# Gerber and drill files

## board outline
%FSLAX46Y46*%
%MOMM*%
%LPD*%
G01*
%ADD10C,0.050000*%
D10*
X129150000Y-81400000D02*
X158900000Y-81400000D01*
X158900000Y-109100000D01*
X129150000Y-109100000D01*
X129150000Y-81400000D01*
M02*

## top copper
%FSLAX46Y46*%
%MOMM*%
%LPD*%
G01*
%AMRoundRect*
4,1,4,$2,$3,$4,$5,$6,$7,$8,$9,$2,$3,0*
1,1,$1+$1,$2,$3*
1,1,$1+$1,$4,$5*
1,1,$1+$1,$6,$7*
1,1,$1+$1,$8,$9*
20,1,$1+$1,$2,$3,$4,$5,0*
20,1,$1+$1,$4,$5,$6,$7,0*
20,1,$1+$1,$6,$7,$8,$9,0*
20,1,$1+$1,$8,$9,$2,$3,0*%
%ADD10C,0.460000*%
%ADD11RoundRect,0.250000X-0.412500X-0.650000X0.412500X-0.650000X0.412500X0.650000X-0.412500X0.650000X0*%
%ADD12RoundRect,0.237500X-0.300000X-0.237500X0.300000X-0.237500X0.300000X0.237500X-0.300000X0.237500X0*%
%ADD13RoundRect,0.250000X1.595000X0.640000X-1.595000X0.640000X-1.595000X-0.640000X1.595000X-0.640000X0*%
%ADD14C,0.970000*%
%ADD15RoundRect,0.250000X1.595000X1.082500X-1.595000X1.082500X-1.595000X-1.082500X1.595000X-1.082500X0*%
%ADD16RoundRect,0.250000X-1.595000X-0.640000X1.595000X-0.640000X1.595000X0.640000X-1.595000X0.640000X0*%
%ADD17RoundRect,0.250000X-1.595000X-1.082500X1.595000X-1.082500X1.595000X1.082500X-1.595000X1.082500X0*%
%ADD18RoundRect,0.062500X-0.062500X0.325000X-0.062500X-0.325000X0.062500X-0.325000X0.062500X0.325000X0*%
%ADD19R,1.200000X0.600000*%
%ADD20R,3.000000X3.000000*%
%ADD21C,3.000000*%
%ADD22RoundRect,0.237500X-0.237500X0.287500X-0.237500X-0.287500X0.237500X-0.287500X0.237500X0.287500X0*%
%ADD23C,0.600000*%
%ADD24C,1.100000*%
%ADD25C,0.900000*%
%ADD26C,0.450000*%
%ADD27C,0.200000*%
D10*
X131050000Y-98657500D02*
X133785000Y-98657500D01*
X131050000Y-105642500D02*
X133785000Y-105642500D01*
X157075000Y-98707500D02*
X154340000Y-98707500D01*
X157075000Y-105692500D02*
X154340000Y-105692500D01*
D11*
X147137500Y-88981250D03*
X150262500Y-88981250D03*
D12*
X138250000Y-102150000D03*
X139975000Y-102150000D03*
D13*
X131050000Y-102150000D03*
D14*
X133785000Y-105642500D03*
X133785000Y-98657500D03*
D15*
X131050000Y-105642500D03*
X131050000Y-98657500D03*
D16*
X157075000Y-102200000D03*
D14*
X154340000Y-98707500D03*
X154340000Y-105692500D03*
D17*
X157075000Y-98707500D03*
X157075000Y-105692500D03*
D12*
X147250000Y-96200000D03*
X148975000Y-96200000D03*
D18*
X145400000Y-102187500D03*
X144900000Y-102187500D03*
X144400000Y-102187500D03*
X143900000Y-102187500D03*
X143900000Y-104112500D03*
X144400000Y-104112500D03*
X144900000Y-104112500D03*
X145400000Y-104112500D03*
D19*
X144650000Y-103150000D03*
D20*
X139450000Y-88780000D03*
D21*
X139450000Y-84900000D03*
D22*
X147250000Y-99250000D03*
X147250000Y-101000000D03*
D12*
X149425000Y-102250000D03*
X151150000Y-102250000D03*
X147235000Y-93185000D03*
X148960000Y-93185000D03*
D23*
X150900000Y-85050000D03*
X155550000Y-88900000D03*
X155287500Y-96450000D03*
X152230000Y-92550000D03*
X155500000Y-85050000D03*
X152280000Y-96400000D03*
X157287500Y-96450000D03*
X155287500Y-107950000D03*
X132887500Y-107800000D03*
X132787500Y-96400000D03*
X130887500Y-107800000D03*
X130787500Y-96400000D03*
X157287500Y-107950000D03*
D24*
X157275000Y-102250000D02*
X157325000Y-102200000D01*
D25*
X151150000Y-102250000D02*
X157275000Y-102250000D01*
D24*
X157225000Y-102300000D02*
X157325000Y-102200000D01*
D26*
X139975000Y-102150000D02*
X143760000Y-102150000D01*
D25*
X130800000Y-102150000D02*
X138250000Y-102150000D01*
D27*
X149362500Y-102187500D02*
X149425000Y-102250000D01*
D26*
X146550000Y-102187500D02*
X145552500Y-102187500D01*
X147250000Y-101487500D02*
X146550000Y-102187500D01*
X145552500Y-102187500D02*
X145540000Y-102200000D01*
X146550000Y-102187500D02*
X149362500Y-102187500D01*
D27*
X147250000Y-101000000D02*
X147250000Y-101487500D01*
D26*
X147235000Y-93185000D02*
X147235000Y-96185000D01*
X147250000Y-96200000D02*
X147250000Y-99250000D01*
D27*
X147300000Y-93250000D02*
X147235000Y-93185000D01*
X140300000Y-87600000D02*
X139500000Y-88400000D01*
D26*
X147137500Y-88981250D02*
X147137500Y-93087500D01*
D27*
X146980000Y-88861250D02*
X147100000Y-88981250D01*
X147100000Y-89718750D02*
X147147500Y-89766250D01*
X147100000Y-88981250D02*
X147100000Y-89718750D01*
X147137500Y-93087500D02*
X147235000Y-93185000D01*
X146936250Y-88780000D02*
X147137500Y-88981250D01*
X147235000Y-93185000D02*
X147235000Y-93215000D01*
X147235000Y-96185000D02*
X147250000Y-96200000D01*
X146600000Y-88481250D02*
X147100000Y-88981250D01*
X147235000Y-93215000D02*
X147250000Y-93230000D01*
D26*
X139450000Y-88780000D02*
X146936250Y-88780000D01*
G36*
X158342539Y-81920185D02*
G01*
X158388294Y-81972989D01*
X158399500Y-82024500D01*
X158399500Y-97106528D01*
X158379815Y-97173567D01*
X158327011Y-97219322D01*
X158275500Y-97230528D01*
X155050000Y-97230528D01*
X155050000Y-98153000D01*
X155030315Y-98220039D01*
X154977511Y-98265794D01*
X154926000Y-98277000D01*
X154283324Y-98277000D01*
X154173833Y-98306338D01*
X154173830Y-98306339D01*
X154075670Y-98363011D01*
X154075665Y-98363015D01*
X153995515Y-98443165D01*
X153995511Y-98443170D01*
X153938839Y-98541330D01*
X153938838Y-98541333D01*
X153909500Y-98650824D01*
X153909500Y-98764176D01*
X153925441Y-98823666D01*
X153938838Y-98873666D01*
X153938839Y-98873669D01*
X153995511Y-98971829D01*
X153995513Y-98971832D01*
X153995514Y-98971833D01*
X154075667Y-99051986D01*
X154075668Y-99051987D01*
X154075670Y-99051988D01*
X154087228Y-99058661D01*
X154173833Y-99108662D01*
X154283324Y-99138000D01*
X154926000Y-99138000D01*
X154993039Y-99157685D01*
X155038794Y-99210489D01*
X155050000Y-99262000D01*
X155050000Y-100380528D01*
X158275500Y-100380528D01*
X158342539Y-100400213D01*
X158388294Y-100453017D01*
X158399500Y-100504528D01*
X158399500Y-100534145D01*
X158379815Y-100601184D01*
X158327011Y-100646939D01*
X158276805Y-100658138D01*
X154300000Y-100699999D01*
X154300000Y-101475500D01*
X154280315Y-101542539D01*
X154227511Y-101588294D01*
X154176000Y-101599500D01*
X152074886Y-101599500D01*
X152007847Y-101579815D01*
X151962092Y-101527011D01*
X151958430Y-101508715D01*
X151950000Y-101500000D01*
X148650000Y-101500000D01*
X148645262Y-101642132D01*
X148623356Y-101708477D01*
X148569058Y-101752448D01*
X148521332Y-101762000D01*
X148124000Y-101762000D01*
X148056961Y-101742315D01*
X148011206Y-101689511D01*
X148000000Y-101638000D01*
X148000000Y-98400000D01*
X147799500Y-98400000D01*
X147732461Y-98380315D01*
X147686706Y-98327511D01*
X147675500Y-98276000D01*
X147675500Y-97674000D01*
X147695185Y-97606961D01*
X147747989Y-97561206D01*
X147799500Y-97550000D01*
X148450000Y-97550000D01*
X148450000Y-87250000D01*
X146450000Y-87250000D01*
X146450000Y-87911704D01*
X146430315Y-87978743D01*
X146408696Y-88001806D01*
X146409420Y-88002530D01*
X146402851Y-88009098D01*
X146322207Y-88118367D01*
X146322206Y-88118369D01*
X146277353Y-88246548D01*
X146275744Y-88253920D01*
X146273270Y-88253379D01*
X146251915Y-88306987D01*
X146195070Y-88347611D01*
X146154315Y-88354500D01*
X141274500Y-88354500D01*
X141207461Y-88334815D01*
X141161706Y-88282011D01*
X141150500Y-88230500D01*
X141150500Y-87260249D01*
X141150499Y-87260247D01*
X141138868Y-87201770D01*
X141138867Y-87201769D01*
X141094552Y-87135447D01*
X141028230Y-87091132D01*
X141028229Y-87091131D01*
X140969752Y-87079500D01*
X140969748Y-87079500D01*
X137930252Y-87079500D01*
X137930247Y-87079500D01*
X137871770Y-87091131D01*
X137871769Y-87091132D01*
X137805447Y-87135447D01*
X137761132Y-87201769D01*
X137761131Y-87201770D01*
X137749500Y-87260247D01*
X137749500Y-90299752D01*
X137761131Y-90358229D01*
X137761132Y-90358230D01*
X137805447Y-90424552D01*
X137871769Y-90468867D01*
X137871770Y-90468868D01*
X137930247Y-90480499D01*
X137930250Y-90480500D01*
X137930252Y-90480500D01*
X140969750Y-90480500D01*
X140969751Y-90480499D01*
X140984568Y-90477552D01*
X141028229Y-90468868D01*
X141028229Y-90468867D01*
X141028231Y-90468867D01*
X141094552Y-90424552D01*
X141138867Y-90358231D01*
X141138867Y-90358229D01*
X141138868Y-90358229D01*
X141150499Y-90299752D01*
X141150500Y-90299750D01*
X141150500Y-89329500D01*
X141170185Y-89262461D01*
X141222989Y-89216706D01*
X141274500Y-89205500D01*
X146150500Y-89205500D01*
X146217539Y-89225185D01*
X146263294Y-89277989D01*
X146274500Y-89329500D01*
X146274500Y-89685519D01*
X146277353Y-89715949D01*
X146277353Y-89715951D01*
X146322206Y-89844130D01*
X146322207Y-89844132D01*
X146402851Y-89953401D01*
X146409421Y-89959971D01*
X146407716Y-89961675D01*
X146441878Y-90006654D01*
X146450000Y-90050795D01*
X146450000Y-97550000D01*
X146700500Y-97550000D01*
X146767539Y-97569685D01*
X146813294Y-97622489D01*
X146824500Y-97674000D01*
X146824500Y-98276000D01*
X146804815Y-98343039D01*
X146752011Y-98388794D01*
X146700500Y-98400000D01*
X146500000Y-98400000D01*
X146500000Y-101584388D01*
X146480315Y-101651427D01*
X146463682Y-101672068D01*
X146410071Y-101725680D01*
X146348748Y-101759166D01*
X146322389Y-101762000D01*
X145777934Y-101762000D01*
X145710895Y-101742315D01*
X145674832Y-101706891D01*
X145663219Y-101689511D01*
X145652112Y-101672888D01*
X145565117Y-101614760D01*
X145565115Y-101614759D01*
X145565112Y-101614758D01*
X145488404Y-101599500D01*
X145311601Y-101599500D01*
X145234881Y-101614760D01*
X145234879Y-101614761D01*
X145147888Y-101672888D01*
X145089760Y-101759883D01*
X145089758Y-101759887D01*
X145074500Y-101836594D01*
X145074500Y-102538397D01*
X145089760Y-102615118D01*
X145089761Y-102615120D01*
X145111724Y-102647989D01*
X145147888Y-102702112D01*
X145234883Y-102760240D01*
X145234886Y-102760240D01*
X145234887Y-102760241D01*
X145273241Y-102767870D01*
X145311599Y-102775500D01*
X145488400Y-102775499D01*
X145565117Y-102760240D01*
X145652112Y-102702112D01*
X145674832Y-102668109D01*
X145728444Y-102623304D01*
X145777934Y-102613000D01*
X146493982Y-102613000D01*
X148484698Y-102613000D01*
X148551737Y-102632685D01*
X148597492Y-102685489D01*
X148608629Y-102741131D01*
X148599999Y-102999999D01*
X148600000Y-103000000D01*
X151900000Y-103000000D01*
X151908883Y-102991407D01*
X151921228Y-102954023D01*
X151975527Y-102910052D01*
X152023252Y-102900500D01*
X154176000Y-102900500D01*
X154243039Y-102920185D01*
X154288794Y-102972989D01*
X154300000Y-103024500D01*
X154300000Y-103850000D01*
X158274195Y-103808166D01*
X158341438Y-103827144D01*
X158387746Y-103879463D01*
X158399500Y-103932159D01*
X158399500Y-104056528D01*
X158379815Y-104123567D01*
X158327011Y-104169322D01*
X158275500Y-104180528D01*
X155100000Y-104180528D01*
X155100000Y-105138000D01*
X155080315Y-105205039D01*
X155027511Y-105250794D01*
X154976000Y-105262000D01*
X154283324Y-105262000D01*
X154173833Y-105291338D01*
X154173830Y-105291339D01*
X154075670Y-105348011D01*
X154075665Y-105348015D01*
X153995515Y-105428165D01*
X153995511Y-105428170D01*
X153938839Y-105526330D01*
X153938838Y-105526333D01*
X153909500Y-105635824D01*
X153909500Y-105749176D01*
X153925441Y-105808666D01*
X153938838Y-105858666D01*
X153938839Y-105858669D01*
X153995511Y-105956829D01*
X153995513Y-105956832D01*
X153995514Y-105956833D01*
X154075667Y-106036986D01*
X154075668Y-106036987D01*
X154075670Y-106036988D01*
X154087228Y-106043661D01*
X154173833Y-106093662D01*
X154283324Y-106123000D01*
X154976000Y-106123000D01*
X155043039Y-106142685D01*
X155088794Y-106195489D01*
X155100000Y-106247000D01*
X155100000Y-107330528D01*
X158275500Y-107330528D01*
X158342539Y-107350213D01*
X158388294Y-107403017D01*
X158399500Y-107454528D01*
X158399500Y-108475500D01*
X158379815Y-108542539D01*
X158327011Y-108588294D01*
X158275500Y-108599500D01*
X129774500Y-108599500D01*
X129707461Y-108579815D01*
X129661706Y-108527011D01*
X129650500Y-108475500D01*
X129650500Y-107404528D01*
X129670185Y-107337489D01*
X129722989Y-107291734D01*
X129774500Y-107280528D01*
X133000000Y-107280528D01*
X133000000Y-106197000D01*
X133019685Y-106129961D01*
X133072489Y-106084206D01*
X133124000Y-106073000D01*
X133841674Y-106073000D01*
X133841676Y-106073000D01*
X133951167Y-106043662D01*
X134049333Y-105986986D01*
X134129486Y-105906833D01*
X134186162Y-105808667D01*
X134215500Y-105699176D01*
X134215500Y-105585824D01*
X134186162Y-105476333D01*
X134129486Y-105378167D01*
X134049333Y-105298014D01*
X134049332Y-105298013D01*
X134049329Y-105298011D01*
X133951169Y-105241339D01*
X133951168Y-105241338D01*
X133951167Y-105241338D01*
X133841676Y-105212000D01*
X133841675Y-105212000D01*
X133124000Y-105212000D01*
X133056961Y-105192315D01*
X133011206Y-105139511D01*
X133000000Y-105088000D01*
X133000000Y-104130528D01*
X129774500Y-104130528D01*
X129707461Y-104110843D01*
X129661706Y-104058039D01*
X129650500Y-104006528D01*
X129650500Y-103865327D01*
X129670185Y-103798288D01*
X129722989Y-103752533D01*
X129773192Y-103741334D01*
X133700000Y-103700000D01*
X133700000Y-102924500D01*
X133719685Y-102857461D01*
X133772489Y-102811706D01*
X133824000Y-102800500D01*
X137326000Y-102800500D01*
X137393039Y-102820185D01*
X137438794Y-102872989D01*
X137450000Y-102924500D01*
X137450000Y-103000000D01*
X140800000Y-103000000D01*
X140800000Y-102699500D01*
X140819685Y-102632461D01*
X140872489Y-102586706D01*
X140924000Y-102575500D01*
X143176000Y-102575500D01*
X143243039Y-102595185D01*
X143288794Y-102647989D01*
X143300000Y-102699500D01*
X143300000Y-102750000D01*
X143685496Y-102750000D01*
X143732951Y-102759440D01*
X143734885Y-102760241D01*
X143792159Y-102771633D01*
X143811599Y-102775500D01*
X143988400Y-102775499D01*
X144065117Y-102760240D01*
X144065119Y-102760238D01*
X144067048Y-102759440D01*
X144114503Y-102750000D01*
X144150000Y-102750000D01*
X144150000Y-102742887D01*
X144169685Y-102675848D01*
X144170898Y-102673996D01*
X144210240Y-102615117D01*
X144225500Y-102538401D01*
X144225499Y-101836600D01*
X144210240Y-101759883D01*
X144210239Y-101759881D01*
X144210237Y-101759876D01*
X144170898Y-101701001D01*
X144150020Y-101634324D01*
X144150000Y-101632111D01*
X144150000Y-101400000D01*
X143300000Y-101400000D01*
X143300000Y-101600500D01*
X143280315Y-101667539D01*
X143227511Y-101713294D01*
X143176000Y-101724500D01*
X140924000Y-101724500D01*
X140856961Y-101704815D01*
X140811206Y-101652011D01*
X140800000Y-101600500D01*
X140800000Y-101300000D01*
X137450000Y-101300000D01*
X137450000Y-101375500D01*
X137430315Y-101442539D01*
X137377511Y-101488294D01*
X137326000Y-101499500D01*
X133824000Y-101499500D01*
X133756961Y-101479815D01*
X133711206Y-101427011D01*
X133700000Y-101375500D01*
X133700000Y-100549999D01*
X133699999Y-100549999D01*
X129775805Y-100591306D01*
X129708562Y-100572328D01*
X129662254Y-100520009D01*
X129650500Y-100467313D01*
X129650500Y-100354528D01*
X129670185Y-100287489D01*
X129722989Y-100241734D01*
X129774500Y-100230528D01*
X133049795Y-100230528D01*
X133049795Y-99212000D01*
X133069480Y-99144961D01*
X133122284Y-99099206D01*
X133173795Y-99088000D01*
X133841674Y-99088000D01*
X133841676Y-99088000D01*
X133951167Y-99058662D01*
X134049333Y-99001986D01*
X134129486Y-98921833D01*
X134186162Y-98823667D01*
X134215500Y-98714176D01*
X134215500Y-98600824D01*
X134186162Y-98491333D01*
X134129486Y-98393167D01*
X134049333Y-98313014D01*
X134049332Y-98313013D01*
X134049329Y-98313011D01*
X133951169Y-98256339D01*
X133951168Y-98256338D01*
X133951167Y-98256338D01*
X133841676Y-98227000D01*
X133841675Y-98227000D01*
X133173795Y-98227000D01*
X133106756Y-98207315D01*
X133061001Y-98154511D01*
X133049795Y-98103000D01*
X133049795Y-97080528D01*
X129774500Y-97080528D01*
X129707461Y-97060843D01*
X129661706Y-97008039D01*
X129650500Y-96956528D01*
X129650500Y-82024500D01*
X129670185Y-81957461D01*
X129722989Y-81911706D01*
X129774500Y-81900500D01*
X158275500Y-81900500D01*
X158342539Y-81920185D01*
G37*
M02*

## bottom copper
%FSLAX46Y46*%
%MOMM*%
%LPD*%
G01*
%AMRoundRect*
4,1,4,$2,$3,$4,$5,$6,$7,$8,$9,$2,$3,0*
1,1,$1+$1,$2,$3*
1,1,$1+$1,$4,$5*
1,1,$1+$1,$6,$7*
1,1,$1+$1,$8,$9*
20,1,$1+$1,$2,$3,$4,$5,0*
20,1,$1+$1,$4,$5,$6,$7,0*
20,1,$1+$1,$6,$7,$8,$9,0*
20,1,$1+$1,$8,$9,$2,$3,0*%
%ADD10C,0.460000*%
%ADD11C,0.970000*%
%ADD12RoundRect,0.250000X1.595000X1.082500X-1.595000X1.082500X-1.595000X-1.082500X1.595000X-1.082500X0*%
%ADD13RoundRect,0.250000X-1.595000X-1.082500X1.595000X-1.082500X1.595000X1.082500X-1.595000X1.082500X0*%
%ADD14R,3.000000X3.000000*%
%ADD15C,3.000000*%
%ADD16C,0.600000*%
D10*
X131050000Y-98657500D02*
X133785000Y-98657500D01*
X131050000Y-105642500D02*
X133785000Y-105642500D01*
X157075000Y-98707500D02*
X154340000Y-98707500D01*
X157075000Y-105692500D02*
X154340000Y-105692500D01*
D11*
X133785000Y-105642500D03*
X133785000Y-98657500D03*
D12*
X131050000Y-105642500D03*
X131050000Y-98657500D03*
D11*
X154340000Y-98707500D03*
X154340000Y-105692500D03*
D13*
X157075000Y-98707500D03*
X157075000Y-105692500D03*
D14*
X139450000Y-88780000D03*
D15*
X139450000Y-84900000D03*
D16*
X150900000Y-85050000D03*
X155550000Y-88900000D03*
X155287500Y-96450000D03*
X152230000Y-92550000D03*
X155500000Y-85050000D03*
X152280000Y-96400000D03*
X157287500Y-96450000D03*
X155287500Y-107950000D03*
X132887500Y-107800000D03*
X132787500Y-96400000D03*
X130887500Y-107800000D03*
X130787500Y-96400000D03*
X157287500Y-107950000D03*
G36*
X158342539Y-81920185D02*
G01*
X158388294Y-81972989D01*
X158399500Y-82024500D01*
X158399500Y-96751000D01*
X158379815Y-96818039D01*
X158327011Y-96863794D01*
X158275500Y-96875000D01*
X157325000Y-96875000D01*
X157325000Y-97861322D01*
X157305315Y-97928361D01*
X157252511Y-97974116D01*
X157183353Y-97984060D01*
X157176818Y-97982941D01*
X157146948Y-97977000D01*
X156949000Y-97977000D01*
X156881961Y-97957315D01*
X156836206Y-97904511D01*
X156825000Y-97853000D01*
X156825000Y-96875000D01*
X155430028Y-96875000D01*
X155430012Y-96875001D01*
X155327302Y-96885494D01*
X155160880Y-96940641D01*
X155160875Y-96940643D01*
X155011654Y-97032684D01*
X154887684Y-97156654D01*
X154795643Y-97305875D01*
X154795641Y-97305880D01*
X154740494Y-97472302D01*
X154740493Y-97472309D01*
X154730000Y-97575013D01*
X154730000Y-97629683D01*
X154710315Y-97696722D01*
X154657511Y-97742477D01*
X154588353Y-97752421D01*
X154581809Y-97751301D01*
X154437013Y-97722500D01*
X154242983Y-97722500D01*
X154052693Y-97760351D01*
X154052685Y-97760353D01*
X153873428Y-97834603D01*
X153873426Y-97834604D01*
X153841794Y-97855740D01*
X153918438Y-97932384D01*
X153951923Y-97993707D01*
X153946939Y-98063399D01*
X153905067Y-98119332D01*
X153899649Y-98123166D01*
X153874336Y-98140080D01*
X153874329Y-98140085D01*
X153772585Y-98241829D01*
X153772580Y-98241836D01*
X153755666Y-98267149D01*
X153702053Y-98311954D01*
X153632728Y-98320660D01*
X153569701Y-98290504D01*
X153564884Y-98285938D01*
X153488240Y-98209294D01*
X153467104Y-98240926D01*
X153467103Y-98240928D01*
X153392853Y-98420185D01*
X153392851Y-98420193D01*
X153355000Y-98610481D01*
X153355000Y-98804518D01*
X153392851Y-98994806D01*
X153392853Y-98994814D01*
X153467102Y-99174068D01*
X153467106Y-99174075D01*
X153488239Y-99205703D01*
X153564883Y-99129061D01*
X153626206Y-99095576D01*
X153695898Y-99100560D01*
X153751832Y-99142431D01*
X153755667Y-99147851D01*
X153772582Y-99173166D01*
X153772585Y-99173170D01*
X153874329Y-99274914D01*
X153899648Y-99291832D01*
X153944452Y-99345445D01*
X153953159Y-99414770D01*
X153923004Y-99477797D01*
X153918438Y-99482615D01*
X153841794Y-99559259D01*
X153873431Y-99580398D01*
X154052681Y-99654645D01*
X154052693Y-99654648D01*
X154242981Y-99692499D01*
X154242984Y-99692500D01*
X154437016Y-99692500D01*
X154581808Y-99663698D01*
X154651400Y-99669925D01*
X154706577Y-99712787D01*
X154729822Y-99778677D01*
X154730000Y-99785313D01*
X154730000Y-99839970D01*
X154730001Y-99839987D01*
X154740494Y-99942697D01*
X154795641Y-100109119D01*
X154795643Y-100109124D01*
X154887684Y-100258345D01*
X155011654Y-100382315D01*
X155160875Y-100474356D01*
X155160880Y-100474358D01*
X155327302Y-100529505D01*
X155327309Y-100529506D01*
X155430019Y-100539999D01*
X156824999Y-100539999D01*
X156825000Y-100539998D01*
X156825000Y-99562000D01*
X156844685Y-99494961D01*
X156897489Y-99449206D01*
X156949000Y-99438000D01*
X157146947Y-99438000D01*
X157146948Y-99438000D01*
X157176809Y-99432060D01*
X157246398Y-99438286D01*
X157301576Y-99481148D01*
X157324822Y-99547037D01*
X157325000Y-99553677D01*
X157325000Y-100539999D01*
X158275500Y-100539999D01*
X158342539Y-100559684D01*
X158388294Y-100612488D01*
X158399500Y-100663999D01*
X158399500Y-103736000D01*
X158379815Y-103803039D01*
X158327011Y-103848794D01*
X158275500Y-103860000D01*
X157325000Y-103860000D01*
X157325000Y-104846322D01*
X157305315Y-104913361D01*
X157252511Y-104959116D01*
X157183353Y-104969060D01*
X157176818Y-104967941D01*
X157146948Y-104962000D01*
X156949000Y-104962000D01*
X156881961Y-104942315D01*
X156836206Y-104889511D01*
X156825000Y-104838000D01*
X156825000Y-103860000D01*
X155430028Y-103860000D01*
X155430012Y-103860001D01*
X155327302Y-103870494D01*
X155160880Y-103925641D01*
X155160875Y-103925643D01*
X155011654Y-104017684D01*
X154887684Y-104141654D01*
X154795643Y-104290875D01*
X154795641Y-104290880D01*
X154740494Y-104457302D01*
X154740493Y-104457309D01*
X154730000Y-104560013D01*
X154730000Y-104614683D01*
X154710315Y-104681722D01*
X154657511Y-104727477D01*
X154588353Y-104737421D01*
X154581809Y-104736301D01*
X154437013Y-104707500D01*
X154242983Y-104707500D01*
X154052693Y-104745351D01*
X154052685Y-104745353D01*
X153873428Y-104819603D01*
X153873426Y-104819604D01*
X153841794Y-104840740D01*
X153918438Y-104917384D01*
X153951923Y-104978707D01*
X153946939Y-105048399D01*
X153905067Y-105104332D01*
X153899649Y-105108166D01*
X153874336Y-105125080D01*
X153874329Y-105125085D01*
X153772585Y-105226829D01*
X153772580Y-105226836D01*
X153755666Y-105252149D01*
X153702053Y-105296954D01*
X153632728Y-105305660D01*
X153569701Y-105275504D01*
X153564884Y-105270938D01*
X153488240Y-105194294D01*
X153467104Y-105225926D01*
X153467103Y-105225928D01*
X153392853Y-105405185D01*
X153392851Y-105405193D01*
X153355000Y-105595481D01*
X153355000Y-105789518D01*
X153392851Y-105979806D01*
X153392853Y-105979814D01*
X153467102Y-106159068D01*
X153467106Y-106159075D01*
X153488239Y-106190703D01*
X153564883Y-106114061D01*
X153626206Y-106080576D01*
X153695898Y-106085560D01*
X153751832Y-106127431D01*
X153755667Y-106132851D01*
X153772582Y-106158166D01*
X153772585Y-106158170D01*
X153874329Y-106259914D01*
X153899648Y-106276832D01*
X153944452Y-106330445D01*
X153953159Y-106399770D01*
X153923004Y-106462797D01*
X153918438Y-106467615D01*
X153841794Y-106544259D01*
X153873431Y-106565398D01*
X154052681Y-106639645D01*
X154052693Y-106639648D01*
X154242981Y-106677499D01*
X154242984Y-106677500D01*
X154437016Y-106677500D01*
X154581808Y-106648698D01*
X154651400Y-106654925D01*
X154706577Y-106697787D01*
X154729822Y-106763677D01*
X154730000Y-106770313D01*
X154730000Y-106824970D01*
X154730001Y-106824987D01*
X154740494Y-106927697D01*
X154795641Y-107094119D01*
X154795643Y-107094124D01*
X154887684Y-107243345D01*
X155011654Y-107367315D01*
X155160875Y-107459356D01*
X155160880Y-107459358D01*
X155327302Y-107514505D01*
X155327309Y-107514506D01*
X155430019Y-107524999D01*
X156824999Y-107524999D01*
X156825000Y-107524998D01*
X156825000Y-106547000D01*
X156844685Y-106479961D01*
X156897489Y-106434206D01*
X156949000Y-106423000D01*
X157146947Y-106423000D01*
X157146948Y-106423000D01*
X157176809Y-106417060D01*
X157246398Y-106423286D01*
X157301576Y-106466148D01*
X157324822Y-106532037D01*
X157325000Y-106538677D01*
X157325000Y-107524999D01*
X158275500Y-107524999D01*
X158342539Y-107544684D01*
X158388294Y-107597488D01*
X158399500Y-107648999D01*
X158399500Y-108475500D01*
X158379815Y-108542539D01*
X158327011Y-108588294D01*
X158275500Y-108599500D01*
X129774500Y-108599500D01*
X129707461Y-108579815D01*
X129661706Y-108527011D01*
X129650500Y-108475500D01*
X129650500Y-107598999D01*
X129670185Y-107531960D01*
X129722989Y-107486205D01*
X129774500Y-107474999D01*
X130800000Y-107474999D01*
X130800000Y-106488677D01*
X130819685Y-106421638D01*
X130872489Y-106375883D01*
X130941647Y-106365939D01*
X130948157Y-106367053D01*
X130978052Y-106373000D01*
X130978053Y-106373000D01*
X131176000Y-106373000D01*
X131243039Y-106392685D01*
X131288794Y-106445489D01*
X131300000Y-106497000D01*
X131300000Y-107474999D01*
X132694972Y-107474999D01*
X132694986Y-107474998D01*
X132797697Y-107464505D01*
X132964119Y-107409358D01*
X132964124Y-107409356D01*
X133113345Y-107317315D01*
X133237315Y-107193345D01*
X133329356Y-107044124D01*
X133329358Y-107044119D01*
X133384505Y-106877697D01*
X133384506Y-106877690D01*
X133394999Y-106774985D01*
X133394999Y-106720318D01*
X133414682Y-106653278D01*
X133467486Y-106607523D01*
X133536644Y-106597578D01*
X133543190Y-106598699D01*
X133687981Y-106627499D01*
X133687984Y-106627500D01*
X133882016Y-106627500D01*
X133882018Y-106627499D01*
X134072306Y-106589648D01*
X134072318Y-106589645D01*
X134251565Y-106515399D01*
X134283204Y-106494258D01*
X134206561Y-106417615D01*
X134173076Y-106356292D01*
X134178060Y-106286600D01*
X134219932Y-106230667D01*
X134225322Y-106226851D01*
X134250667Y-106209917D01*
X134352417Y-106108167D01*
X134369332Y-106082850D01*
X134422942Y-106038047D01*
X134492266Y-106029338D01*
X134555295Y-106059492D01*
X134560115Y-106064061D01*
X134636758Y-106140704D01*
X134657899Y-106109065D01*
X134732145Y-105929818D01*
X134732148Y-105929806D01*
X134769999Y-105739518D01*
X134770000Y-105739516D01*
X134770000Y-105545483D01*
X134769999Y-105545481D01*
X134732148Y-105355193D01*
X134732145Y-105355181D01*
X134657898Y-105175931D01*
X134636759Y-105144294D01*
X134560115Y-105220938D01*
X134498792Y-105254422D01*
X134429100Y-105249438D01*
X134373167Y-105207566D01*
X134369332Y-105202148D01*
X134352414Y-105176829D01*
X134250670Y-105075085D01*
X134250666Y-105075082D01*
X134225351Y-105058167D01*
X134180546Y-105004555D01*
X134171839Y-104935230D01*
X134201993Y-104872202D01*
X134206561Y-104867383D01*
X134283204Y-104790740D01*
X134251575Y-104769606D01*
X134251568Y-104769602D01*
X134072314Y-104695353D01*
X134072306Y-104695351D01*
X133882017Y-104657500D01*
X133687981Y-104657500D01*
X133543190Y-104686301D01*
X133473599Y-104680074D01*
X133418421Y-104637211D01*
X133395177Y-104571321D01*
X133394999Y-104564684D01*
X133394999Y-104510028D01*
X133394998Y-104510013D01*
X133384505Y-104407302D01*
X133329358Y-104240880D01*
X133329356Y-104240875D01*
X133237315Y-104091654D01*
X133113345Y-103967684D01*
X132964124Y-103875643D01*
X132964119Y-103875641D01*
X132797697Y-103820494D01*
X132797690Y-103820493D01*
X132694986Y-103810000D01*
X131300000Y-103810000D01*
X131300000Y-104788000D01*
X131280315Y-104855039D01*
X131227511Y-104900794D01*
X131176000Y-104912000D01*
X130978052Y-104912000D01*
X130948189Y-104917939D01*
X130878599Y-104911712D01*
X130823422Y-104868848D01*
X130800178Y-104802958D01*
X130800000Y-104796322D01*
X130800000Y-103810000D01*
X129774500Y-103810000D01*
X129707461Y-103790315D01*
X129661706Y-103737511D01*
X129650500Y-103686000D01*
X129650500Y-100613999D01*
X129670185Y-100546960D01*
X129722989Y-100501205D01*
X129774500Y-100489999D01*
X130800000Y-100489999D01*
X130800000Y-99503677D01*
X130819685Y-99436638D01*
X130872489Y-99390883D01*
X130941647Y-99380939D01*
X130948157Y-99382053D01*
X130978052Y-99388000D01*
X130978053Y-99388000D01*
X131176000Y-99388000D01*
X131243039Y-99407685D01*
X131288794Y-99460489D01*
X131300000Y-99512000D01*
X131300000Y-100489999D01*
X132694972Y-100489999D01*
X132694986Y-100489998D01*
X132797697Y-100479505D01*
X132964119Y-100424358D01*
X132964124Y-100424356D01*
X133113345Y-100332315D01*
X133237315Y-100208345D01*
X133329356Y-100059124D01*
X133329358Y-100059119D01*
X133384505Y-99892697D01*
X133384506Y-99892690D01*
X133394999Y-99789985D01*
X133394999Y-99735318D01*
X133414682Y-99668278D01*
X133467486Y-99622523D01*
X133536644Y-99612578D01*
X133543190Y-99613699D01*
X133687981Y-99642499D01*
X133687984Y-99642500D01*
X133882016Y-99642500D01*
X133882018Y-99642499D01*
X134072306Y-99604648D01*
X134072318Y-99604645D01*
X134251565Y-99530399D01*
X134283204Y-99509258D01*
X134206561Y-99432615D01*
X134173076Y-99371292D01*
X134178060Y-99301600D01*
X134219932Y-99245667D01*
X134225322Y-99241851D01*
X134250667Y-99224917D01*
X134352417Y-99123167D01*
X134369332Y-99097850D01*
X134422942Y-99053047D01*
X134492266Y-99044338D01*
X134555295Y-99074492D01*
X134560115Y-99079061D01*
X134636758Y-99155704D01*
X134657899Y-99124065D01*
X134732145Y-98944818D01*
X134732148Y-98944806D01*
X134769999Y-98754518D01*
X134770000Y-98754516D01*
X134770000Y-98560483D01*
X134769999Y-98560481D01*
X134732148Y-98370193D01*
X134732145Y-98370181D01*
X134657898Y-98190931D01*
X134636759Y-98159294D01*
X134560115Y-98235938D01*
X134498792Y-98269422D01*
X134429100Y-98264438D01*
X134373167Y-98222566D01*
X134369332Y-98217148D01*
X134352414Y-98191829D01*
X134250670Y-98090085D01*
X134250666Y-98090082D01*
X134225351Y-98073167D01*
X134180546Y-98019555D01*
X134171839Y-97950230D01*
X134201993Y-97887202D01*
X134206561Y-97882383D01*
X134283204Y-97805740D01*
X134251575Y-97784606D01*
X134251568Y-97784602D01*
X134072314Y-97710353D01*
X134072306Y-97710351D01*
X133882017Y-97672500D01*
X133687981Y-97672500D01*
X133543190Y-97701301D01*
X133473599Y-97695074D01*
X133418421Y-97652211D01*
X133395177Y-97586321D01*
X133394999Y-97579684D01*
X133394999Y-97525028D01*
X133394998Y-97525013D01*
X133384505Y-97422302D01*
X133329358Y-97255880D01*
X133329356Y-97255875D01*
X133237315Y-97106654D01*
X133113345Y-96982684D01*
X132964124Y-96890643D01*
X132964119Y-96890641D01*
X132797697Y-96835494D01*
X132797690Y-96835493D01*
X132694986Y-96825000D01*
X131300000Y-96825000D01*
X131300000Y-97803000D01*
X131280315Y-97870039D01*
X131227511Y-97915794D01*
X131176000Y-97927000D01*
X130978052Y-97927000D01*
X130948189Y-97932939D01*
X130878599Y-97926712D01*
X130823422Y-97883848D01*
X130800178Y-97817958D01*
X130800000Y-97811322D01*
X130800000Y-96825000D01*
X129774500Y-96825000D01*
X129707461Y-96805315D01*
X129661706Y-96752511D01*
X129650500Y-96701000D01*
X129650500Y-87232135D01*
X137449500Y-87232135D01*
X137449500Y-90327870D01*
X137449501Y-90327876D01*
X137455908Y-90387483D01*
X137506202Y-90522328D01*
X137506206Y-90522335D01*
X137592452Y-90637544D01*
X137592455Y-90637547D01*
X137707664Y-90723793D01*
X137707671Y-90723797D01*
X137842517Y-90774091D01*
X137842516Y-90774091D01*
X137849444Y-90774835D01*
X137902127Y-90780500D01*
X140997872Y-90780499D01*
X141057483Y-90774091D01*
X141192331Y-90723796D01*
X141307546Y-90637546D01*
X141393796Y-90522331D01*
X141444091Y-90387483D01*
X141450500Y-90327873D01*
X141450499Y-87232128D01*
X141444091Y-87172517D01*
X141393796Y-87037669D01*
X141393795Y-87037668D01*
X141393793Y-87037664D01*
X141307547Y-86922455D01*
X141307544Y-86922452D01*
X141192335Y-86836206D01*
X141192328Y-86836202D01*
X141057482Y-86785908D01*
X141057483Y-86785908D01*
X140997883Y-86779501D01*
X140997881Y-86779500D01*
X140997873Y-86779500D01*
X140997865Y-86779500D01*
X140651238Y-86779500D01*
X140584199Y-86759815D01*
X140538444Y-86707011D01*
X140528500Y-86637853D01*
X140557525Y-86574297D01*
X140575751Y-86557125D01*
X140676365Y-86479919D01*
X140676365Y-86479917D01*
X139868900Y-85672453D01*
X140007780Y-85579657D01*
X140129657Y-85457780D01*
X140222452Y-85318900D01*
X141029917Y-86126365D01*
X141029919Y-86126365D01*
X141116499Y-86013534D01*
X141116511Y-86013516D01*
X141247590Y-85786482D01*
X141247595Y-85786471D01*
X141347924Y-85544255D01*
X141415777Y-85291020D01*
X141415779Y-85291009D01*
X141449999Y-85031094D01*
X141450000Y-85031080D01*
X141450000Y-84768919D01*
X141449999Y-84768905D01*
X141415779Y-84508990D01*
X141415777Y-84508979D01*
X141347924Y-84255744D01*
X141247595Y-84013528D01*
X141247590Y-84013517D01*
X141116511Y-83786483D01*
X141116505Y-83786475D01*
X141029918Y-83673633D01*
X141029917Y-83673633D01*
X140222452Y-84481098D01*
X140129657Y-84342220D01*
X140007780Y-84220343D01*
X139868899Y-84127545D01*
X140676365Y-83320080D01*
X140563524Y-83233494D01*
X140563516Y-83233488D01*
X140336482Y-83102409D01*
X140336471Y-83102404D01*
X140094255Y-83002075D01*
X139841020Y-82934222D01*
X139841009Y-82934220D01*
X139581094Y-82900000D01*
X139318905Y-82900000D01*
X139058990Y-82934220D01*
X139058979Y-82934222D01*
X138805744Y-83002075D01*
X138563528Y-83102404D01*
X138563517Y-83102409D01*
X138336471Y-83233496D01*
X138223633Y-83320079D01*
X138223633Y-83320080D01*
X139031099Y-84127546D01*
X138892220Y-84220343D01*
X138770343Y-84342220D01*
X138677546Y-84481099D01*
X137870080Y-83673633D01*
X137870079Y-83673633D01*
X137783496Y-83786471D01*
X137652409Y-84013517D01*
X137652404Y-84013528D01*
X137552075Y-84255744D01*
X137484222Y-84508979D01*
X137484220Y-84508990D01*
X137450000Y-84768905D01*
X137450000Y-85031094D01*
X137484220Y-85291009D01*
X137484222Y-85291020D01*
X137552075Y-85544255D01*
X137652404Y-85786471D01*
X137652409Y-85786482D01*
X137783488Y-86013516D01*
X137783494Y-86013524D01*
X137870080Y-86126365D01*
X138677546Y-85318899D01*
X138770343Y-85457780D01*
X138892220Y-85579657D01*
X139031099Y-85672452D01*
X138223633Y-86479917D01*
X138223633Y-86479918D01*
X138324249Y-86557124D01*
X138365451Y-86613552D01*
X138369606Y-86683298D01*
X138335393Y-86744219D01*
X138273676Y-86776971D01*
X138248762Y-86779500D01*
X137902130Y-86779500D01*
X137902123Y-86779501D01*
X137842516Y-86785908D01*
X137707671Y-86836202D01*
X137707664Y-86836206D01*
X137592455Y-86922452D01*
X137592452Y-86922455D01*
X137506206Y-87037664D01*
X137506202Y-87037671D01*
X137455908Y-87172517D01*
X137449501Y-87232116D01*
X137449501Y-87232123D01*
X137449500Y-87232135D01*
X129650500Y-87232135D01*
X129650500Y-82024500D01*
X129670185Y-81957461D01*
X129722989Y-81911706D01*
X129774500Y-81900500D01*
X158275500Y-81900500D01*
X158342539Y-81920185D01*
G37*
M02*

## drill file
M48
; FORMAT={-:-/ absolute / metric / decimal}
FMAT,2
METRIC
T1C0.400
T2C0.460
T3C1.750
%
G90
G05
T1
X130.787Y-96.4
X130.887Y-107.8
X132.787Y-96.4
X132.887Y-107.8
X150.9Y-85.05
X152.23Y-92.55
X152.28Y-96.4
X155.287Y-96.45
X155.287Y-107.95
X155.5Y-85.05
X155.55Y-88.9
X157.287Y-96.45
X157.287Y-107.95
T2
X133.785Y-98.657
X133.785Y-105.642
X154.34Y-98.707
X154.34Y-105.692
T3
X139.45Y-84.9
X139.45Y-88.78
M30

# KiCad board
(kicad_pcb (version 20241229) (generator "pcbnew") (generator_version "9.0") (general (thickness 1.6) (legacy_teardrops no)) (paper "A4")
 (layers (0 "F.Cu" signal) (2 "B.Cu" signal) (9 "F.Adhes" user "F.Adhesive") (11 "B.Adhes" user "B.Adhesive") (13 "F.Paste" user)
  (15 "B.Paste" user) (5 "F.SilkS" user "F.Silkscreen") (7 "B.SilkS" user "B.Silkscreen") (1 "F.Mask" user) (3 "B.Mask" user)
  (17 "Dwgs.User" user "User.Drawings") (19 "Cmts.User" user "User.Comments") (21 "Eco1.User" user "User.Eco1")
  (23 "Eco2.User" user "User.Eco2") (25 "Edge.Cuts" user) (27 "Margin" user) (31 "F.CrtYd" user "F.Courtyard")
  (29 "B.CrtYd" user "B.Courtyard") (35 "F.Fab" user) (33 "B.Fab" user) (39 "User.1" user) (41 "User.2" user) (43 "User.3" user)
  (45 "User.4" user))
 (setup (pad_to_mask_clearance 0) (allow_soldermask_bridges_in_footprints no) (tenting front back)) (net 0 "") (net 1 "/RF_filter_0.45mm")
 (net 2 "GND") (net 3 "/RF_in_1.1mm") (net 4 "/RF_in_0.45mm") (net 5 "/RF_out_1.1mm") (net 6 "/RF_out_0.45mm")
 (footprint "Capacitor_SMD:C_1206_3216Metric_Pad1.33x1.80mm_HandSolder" (layer "F.Cu") (at 148.7 88.98125)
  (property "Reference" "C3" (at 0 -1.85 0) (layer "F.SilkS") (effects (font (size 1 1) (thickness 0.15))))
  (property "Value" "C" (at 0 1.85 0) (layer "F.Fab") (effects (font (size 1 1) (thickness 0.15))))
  (pad "1" smd roundrect (at -1.5625 0) (size 1.325 1.8) (layers "F.Cu" "F.Mask" "F.Paste") (roundrect_rratio 0.188679)
   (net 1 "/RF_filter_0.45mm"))
  (pad "2" smd roundrect (at 1.5625 0) (size 1.325 1.8) (layers "F.Cu" "F.Mask" "F.Paste") (roundrect_rratio 0.188679) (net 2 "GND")))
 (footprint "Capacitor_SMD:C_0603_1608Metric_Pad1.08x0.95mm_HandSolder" (layer "F.Cu") (at 139.1125 102.15)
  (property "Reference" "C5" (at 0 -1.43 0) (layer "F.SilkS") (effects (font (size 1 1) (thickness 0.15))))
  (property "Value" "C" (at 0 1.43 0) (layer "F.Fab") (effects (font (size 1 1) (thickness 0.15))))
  (pad "1" smd roundrect (at -0.8625 0) (size 1.075 0.95) (layers "F.Cu" "F.Mask" "F.Paste") (roundrect_rratio 0.25) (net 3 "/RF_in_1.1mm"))
  (pad "2" smd roundrect (at 0.8625 0) (size 1.075 0.95) (layers "F.Cu" "F.Mask" "F.Paste") (roundrect_rratio 0.25) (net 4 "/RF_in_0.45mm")))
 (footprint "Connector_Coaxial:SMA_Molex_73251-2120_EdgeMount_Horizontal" (layer "F.Cu") (at 130.8 102.15 180)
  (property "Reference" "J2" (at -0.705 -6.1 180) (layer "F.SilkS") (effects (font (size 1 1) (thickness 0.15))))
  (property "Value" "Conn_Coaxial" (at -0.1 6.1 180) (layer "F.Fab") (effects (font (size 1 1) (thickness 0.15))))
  (fp_line (start -0.25 3.4925) (end -2.985 3.4925) (stroke (width 0.46) (type default)) (layer "F.Cu"))
  (fp_line (start -0.25 -3.4925) (end -2.985 -3.4925) (stroke (width 0.46) (type default)) (layer "F.Cu"))
  (fp_line (start -0.25 3.4925) (end -2.985 3.4925) (stroke (width 0.46) (type default)) (layer "B.Cu"))
  (fp_line (start -0.25 -3.4925) (end -2.985 -3.4925) (stroke (width 0.46) (type default)) (layer "B.Cu"))
  (pad "1" smd roundrect (at -0.25 0 180) (size 3.69 1.78) (layers "F.Cu" "F.Mask" "F.Paste") (roundrect_rratio 0.1404494382)
   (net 3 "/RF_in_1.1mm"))
  (pad "2" thru_hole circle (at -2.985 -3.4925 180) (size 0.97 0.97) (drill 0.46) (layers "*.Cu") (remove_unused_layers no) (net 2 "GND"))
  (pad "2" thru_hole circle (at -2.985 3.4925 180) (size 0.97 0.97) (drill 0.46) (layers "*.Cu") (remove_unused_layers no) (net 2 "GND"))
  (pad "2" smd roundrect (at -0.25 -3.4925 180) (size 3.69 2.665) (layers "F.Cu" "F.Mask" "F.Paste") (roundrect_rratio 0.09380863039)
   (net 2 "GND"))
  (pad "2" smd roundrect (at -0.25 -3.4925 180) (size 3.69 2.665) (layers "B.Cu" "B.Mask" "B.Paste") (roundrect_rratio 0.09380863039)
   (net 2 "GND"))
  (pad "2" smd roundrect (at -0.25 3.4925 180) (size 3.69 2.665) (layers "F.Cu" "F.Mask" "F.Paste") (roundrect_rratio 0.09380863039)
   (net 2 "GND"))
  (pad "2" smd roundrect (at -0.25 3.4925 180) (size 3.69 2.665) (layers "B.Cu" "B.Mask" "B.Paste") (roundrect_rratio 0.09380863039)
   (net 2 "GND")))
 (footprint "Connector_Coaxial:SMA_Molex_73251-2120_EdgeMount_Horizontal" (layer "F.Cu") (at 157.325 102.2)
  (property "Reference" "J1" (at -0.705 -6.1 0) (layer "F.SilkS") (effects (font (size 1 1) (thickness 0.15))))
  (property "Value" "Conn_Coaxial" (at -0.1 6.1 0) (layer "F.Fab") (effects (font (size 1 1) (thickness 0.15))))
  (fp_line (start -0.25 -3.4925) (end -2.985 -3.4925) (stroke (width 0.46) (type default)) (layer "F.Cu"))
  (fp_line (start -0.25 3.4925) (end -2.985 3.4925) (stroke (width 0.46) (type default)) (layer "F.Cu"))
  (fp_line (start -0.25 -3.4925) (end -2.985 -3.4925) (stroke (width 0.46) (type default)) (layer "B.Cu"))
  (fp_line (start -0.25 3.4925) (end -2.985 3.4925) (stroke (width 0.46) (type default)) (layer "B.Cu"))
  (pad "1" smd roundrect (at -0.25 0) (size 3.69 1.78) (layers "F.Cu" "F.Mask" "F.Paste") (roundrect_rratio 0.1404494382)
   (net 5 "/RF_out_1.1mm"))
  (pad "2" thru_hole circle (at -2.985 -3.4925) (size 0.97 0.97) (drill 0.46) (layers "*.Cu") (remove_unused_layers no) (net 2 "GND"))
  (pad "2" thru_hole circle (at -2.985 3.4925) (size 0.97 0.97) (drill 0.46) (layers "*.Cu") (remove_unused_layers no) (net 2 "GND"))
  (pad "2" smd roundrect (at -0.25 -3.4925) (size 3.69 2.665) (layers "F.Cu" "F.Mask" "F.Paste") (roundrect_rratio 0.09380863039)
   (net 2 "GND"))
  (pad "2" smd roundrect (at -0.25 -3.4925) (size 3.69 2.665) (layers "B.Cu" "B.Mask" "B.Paste") (roundrect_rratio 0.09380863039)
   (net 2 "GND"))
  (pad "2" smd roundrect (at -0.25 3.4925) (size 3.69 2.665) (layers "F.Cu" "F.Mask" "F.Paste") (roundrect_rratio 0.09380863039)
   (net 2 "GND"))
  (pad "2" smd roundrect (at -0.25 3.4925) (size 3.69 2.665) (layers "B.Cu" "B.Mask" "B.Paste") (roundrect_rratio 0.09380863039)
   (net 2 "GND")))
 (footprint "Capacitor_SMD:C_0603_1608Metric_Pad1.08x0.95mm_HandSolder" (layer "F.Cu") (at 148.1125 96.2)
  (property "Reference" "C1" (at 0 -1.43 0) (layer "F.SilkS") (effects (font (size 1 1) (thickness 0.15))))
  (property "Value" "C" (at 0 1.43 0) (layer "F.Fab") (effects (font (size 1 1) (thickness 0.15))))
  (pad "1" smd roundrect (at -0.8625 0) (size 1.075 0.95) (layers "F.Cu" "F.Mask" "F.Paste") (roundrect_rratio 0.25)
   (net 1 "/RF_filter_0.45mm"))
  (pad "2" smd roundrect (at 0.8625 0) (size 1.075 0.95) (layers "F.Cu" "F.Mask" "F.Paste") (roundrect_rratio 0.25) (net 2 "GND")))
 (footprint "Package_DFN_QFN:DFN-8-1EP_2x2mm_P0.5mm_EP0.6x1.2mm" (layer "F.Cu") (at 144.65 103.15 -90)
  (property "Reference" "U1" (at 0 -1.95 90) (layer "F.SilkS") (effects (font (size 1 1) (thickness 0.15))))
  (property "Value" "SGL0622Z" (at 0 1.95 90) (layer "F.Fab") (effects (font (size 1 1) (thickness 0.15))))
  (pad "" smd roundrect (at -0.15 -0.3 270) (size 0.24 0.48) (layers "F.Paste") (roundrect_rratio 0.25))
  (pad "" smd roundrect (at -0.15 0.3 270) (size 0.24 0.48) (layers "F.Paste") (roundrect_rratio 0.25))
  (pad "" smd roundrect (at 0.15 -0.3 270) (size 0.24 0.48) (layers "F.Paste") (roundrect_rratio 0.25))
  (pad "" smd roundrect (at 0.15 0.3 270) (size 0.24 0.48) (layers "F.Paste") (roundrect_rratio 0.25))
  (pad "1" smd roundrect (at -0.9625 -0.75 270) (size 0.775 0.25) (layers "F.Cu" "F.Mask" "F.Paste") (roundrect_rratio 0.25)
   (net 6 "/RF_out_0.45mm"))
  (pad "2" smd roundrect (at -0.9625 -0.25 270) (size 0.775 0.25) (layers "F.Cu" "F.Mask" "F.Paste") (roundrect_rratio 0.25) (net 2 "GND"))
  (pad "3" smd roundrect (at -0.9625 0.25 270) (size 0.775 0.25) (layers "F.Cu" "F.Mask" "F.Paste") (roundrect_rratio 0.25) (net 2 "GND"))
  (pad "4" smd roundrect (at -0.9625 0.75 270) (size 0.775 0.25) (layers "F.Cu" "F.Mask" "F.Paste") (roundrect_rratio 0.25)
   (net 4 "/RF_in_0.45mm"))
  (pad "5" smd roundrect (at 0.9625 0.75 270) (size 0.775 0.25) (layers "F.Cu" "F.Mask" "F.Paste") (roundrect_rratio 0.25) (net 2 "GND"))
  (pad "6" smd roundrect (at 0.9625 0.25 270) (size 0.775 0.25) (layers "F.Cu" "F.Mask" "F.Paste") (roundrect_rratio 0.25) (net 2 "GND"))
  (pad "7" smd roundrect (at 0.9625 -0.25 270) (size 0.775 0.25) (layers "F.Cu" "F.Mask" "F.Paste") (roundrect_rratio 0.25) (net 2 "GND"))
  (pad "8" smd roundrect (at 0.9625 -0.75 270) (size 0.775 0.25) (layers "F.Cu" "F.Mask" "F.Paste") (roundrect_rratio 0.25) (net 2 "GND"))
  (pad "9" smd rect (at 0 0 270) (size 0.6 1.2) (layers "F.Cu" "F.Mask") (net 2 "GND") (zone_connect 2)))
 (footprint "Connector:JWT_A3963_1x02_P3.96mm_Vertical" (layer "F.Cu") (at 139.45 88.78 90)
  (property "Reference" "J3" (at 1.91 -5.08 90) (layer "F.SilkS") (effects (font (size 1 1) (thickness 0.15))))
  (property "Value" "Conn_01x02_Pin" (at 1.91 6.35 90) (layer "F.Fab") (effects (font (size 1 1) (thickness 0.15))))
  (pad "1" thru_hole rect (at 0 0 90) (size 3 3) (drill 1.75) (layers "*.Cu" "*.Mask") (remove_unused_layers no) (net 1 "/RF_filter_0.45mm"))
  (pad "2" thru_hole circle (at 3.88 0 90) (size 3 3) (drill 1.75) (layers "*.Cu" "*.Mask") (remove_unused_layers no) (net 2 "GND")))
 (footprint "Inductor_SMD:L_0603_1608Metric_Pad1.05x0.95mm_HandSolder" (layer "F.Cu") (at 147.25 100.125 -90)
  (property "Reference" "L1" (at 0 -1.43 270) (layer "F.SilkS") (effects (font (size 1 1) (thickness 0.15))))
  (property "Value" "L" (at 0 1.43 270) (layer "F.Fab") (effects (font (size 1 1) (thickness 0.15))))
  (pad "1" smd roundrect (at -0.875 0 270) (size 1.05 0.95) (layers "F.Cu" "F.Mask" "F.Paste") (roundrect_rratio 0.25)
   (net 1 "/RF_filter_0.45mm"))
  (pad "2" smd roundrect (at 0.875 0 270) (size 1.05 0.95) (layers "F.Cu" "F.Mask" "F.Paste") (roundrect_rratio 0.25)
   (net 6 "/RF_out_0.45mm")))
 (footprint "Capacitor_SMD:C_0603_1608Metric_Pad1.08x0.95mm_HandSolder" (layer "F.Cu") (at 150.2875 102.25)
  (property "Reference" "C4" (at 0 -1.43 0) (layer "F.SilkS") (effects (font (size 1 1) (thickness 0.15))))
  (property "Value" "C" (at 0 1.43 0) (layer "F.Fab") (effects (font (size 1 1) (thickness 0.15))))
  (pad "1" smd roundrect (at -0.8625 0) (size 1.075 0.95) (layers "F.Cu" "F.Mask" "F.Paste") (roundrect_rratio 0.25)
   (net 6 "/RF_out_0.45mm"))
  (pad "2" smd roundrect (at 0.8625 0) (size 1.075 0.95) (layers "F.Cu" "F.Mask" "F.Paste") (roundrect_rratio 0.25) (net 5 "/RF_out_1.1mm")))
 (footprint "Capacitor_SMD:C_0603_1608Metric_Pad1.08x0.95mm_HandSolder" (layer "F.Cu") (at 148.0975 93.185)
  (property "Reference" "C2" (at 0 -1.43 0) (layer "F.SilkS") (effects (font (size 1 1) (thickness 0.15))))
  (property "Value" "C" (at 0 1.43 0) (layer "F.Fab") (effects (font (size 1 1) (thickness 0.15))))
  (pad "1" smd roundrect (at -0.8625 0) (size 1.075 0.95) (layers "F.Cu" "F.Mask" "F.Paste") (roundrect_rratio 0.25)
   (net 1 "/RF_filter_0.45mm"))
  (pad "2" smd roundrect (at 0.8625 0) (size 1.075 0.95) (layers "F.Cu" "F.Mask" "F.Paste") (roundrect_rratio 0.25) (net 2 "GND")))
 (gr_rect (start 129.15 81.4) (end 158.9 109.1) (stroke (width 0.05) (type solid)) (fill no) (layer "Edge.Cuts"))
 (via (at 150.9 85.05) (size 0.6) (drill 0.4) (layers "F.Cu" "B.Cu") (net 2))
 (via (at 155.55 88.9) (size 0.6) (drill 0.4) (layers "F.Cu" "B.Cu") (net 2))
 (via (at 155.2875 96.45) (size 0.6) (drill 0.4) (layers "F.Cu" "B.Cu") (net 2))
 (via (at 152.23 92.55) (size 0.6) (drill 0.4) (layers "F.Cu" "B.Cu") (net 2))
 (via (at 155.5 85.05) (size 0.6) (drill 0.4) (layers "F.Cu" "B.Cu") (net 2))
 (via (at 152.28 96.4) (size 0.6) (drill 0.4) (layers "F.Cu" "B.Cu") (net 2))
 (via (at 157.2875 96.45) (size 0.6) (drill 0.4) (layers "F.Cu" "B.Cu") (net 2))
 (via (at 155.2875 107.95) (size 0.6) (drill 0.4) (layers "F.Cu" "B.Cu") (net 2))
 (via (at 132.8875 107.8) (size 0.6) (drill 0.4) (layers "F.Cu" "B.Cu") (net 2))
 (via (at 132.7875 96.4) (size 0.6) (drill 0.4) (layers "F.Cu" "B.Cu") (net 2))
 (via (at 130.8875 107.8) (size 0.6) (drill 0.4) (layers "F.Cu" "B.Cu") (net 2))
 (via (at 130.7875 96.4) (size 0.6) (drill 0.4) (layers "F.Cu" "B.Cu") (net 2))
 (via (at 157.2875 107.95) (size 0.6) (drill 0.4) (layers "F.Cu" "B.Cu") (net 2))
 (segment (start 157.275 102.25) (end 157.325 102.2) (width 1.1) (layer "F.Cu") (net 5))
 (segment (start 151.15 102.25) (end 157.275 102.25) (width 0.9) (layer "F.Cu") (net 5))
 (segment (start 157.225 102.3) (end 157.325 102.2) (width 1.1) (layer "F.Cu") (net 5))
 (segment (start 139.975 102.15) (end 143.76 102.15) (width 0.45) (layer "F.Cu") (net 4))
 (segment (start 130.8 102.15) (end 138.25 102.15) (width 0.9) (layer "F.Cu") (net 3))
 (segment (start 149.3625 102.1875) (end 149.425 102.25) (width 0.2) (layer "F.Cu") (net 6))
 (segment (start 146.55 102.1875) (end 145.5525 102.1875) (width 0.45) (layer "F.Cu") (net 6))
 (segment (start 147.25 101.4875) (end 146.55 102.1875) (width 0.45) (layer "F.Cu") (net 6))
 (segment (start 145.5525 102.1875) (end 145.54 102.2) (width 0.45) (layer "F.Cu") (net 6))
 (segment (start 146.55 102.1875) (end 149.3625 102.1875) (width 0.45) (layer "F.Cu") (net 6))
 (segment (start 147.25 101) (end 147.25 101.4875) (width 0.2) (layer "F.Cu") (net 6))
 (segment (start 147.235 93.185) (end 147.235 96.185) (width 0.45) (layer "F.Cu") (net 1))
 (segment (start 147.25 96.2) (end 147.25 99.25) (width 0.45) (layer "F.Cu") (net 1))
 (segment (start 147.3 93.25) (end 147.235 93.185) (width 0.2) (layer "F.Cu") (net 1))
 (segment (start 140.3 87.6) (end 139.5 88.4) (width 0.2) (layer "F.Cu") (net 1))
 (segment (start 147.1375 88.98125) (end 147.1375 93.0875) (width 0.45) (layer "F.Cu") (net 1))
 (segment (start 146.98 88.86125) (end 147.1 88.98125) (width 0.2) (layer "F.Cu") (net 1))
 (segment (start 147.1 89.71875) (end 147.1475 89.76625) (width 0.2) (layer "F.Cu") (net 1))
 (segment (start 147.1 88.98125) (end 147.1 89.71875) (width 0.2) (layer "F.Cu") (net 1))
 (segment (start 147.1375 93.0875) (end 147.235 93.185) (width 0.2) (layer "F.Cu") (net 1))
 (segment (start 146.93625 88.78) (end 147.1375 88.98125) (width 0.2) (layer "F.Cu") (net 1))
 (segment (start 147.235 93.185) (end 147.235 93.215) (width 0.2) (layer "F.Cu") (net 1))
 (segment (start 147.235 96.185) (end 147.25 96.2) (width 0.2) (layer "F.Cu") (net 1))
 (segment (start 146.6 88.48125) (end 147.1 88.98125) (width 0.2) (layer "F.Cu") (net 1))
 (segment (start 147.235 93.215) (end 147.25 93.23) (width 0.2) (layer "F.Cu") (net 1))
 (segment (start 139.45 88.78) (end 146.93625 88.78) (width 0.45) (layer "F.Cu") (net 1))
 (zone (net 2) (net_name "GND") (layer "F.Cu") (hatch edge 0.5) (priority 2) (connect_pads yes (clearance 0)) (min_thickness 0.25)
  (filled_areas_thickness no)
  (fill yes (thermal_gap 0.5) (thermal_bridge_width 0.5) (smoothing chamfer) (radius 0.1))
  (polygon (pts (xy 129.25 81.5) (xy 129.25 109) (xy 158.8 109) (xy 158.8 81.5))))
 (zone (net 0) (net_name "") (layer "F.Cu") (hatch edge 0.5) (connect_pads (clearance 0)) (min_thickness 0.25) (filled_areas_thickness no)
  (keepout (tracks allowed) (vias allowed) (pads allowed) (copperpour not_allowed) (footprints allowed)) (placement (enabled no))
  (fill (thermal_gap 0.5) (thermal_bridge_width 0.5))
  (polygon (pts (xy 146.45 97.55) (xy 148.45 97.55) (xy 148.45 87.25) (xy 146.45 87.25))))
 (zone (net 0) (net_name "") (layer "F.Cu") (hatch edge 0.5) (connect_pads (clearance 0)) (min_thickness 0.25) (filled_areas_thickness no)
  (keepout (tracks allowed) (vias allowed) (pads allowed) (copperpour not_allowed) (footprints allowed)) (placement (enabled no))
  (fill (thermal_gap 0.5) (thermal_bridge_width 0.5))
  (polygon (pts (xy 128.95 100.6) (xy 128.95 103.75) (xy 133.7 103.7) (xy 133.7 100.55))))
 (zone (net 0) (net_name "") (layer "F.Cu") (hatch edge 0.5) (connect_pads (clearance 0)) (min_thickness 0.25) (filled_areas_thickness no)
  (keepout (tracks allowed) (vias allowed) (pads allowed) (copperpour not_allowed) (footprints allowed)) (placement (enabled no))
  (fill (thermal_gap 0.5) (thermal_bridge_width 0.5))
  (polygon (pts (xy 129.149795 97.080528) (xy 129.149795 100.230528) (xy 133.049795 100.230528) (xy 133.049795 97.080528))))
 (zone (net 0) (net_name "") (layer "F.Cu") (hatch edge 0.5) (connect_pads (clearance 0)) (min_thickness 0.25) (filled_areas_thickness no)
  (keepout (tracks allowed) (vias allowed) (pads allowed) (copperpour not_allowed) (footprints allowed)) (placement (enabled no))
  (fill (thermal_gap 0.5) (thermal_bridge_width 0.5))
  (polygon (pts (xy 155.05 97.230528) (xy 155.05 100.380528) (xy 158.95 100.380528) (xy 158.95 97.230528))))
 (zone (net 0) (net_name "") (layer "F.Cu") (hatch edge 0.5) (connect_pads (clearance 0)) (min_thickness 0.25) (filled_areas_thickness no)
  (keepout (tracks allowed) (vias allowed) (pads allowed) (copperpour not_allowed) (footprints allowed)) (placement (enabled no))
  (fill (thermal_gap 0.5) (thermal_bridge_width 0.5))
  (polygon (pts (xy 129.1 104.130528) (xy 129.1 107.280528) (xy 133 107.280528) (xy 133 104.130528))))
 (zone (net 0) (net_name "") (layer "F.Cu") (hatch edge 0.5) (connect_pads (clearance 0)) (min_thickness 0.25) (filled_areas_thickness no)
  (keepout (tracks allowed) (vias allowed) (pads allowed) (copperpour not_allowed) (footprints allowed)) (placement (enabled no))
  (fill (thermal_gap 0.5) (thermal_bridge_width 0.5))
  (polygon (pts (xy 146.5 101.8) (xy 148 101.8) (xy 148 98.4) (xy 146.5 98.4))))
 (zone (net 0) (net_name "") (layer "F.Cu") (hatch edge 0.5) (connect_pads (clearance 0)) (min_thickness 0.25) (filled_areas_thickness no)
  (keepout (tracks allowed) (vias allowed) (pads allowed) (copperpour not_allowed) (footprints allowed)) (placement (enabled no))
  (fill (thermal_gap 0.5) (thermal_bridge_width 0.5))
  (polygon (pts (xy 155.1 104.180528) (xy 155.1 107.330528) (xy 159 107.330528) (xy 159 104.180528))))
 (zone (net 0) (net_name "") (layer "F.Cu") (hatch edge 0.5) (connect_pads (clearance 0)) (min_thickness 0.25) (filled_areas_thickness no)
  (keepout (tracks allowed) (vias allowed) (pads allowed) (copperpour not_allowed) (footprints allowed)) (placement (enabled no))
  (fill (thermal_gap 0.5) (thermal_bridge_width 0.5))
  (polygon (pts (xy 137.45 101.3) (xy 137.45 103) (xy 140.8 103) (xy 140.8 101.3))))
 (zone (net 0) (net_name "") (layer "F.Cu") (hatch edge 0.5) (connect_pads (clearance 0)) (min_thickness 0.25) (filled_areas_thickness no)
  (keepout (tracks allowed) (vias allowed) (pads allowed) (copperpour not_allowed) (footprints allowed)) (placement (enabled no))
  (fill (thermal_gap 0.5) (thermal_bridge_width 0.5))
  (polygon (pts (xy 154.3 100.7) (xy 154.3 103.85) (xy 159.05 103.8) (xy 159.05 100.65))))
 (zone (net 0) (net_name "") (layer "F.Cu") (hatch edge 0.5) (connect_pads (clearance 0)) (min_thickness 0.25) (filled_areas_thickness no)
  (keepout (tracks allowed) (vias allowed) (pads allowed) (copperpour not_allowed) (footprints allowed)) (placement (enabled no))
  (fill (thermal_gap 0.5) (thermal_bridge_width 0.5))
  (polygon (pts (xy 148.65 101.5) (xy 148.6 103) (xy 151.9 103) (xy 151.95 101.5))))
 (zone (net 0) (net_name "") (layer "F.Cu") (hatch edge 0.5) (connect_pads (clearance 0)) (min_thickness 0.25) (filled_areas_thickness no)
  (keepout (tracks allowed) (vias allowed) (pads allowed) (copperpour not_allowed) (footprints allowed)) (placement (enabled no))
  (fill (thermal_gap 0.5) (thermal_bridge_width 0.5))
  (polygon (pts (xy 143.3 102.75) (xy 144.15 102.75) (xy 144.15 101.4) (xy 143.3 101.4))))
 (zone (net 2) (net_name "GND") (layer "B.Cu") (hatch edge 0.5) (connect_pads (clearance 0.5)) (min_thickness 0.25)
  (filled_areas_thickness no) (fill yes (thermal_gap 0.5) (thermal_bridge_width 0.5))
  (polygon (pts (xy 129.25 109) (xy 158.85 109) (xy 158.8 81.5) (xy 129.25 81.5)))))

